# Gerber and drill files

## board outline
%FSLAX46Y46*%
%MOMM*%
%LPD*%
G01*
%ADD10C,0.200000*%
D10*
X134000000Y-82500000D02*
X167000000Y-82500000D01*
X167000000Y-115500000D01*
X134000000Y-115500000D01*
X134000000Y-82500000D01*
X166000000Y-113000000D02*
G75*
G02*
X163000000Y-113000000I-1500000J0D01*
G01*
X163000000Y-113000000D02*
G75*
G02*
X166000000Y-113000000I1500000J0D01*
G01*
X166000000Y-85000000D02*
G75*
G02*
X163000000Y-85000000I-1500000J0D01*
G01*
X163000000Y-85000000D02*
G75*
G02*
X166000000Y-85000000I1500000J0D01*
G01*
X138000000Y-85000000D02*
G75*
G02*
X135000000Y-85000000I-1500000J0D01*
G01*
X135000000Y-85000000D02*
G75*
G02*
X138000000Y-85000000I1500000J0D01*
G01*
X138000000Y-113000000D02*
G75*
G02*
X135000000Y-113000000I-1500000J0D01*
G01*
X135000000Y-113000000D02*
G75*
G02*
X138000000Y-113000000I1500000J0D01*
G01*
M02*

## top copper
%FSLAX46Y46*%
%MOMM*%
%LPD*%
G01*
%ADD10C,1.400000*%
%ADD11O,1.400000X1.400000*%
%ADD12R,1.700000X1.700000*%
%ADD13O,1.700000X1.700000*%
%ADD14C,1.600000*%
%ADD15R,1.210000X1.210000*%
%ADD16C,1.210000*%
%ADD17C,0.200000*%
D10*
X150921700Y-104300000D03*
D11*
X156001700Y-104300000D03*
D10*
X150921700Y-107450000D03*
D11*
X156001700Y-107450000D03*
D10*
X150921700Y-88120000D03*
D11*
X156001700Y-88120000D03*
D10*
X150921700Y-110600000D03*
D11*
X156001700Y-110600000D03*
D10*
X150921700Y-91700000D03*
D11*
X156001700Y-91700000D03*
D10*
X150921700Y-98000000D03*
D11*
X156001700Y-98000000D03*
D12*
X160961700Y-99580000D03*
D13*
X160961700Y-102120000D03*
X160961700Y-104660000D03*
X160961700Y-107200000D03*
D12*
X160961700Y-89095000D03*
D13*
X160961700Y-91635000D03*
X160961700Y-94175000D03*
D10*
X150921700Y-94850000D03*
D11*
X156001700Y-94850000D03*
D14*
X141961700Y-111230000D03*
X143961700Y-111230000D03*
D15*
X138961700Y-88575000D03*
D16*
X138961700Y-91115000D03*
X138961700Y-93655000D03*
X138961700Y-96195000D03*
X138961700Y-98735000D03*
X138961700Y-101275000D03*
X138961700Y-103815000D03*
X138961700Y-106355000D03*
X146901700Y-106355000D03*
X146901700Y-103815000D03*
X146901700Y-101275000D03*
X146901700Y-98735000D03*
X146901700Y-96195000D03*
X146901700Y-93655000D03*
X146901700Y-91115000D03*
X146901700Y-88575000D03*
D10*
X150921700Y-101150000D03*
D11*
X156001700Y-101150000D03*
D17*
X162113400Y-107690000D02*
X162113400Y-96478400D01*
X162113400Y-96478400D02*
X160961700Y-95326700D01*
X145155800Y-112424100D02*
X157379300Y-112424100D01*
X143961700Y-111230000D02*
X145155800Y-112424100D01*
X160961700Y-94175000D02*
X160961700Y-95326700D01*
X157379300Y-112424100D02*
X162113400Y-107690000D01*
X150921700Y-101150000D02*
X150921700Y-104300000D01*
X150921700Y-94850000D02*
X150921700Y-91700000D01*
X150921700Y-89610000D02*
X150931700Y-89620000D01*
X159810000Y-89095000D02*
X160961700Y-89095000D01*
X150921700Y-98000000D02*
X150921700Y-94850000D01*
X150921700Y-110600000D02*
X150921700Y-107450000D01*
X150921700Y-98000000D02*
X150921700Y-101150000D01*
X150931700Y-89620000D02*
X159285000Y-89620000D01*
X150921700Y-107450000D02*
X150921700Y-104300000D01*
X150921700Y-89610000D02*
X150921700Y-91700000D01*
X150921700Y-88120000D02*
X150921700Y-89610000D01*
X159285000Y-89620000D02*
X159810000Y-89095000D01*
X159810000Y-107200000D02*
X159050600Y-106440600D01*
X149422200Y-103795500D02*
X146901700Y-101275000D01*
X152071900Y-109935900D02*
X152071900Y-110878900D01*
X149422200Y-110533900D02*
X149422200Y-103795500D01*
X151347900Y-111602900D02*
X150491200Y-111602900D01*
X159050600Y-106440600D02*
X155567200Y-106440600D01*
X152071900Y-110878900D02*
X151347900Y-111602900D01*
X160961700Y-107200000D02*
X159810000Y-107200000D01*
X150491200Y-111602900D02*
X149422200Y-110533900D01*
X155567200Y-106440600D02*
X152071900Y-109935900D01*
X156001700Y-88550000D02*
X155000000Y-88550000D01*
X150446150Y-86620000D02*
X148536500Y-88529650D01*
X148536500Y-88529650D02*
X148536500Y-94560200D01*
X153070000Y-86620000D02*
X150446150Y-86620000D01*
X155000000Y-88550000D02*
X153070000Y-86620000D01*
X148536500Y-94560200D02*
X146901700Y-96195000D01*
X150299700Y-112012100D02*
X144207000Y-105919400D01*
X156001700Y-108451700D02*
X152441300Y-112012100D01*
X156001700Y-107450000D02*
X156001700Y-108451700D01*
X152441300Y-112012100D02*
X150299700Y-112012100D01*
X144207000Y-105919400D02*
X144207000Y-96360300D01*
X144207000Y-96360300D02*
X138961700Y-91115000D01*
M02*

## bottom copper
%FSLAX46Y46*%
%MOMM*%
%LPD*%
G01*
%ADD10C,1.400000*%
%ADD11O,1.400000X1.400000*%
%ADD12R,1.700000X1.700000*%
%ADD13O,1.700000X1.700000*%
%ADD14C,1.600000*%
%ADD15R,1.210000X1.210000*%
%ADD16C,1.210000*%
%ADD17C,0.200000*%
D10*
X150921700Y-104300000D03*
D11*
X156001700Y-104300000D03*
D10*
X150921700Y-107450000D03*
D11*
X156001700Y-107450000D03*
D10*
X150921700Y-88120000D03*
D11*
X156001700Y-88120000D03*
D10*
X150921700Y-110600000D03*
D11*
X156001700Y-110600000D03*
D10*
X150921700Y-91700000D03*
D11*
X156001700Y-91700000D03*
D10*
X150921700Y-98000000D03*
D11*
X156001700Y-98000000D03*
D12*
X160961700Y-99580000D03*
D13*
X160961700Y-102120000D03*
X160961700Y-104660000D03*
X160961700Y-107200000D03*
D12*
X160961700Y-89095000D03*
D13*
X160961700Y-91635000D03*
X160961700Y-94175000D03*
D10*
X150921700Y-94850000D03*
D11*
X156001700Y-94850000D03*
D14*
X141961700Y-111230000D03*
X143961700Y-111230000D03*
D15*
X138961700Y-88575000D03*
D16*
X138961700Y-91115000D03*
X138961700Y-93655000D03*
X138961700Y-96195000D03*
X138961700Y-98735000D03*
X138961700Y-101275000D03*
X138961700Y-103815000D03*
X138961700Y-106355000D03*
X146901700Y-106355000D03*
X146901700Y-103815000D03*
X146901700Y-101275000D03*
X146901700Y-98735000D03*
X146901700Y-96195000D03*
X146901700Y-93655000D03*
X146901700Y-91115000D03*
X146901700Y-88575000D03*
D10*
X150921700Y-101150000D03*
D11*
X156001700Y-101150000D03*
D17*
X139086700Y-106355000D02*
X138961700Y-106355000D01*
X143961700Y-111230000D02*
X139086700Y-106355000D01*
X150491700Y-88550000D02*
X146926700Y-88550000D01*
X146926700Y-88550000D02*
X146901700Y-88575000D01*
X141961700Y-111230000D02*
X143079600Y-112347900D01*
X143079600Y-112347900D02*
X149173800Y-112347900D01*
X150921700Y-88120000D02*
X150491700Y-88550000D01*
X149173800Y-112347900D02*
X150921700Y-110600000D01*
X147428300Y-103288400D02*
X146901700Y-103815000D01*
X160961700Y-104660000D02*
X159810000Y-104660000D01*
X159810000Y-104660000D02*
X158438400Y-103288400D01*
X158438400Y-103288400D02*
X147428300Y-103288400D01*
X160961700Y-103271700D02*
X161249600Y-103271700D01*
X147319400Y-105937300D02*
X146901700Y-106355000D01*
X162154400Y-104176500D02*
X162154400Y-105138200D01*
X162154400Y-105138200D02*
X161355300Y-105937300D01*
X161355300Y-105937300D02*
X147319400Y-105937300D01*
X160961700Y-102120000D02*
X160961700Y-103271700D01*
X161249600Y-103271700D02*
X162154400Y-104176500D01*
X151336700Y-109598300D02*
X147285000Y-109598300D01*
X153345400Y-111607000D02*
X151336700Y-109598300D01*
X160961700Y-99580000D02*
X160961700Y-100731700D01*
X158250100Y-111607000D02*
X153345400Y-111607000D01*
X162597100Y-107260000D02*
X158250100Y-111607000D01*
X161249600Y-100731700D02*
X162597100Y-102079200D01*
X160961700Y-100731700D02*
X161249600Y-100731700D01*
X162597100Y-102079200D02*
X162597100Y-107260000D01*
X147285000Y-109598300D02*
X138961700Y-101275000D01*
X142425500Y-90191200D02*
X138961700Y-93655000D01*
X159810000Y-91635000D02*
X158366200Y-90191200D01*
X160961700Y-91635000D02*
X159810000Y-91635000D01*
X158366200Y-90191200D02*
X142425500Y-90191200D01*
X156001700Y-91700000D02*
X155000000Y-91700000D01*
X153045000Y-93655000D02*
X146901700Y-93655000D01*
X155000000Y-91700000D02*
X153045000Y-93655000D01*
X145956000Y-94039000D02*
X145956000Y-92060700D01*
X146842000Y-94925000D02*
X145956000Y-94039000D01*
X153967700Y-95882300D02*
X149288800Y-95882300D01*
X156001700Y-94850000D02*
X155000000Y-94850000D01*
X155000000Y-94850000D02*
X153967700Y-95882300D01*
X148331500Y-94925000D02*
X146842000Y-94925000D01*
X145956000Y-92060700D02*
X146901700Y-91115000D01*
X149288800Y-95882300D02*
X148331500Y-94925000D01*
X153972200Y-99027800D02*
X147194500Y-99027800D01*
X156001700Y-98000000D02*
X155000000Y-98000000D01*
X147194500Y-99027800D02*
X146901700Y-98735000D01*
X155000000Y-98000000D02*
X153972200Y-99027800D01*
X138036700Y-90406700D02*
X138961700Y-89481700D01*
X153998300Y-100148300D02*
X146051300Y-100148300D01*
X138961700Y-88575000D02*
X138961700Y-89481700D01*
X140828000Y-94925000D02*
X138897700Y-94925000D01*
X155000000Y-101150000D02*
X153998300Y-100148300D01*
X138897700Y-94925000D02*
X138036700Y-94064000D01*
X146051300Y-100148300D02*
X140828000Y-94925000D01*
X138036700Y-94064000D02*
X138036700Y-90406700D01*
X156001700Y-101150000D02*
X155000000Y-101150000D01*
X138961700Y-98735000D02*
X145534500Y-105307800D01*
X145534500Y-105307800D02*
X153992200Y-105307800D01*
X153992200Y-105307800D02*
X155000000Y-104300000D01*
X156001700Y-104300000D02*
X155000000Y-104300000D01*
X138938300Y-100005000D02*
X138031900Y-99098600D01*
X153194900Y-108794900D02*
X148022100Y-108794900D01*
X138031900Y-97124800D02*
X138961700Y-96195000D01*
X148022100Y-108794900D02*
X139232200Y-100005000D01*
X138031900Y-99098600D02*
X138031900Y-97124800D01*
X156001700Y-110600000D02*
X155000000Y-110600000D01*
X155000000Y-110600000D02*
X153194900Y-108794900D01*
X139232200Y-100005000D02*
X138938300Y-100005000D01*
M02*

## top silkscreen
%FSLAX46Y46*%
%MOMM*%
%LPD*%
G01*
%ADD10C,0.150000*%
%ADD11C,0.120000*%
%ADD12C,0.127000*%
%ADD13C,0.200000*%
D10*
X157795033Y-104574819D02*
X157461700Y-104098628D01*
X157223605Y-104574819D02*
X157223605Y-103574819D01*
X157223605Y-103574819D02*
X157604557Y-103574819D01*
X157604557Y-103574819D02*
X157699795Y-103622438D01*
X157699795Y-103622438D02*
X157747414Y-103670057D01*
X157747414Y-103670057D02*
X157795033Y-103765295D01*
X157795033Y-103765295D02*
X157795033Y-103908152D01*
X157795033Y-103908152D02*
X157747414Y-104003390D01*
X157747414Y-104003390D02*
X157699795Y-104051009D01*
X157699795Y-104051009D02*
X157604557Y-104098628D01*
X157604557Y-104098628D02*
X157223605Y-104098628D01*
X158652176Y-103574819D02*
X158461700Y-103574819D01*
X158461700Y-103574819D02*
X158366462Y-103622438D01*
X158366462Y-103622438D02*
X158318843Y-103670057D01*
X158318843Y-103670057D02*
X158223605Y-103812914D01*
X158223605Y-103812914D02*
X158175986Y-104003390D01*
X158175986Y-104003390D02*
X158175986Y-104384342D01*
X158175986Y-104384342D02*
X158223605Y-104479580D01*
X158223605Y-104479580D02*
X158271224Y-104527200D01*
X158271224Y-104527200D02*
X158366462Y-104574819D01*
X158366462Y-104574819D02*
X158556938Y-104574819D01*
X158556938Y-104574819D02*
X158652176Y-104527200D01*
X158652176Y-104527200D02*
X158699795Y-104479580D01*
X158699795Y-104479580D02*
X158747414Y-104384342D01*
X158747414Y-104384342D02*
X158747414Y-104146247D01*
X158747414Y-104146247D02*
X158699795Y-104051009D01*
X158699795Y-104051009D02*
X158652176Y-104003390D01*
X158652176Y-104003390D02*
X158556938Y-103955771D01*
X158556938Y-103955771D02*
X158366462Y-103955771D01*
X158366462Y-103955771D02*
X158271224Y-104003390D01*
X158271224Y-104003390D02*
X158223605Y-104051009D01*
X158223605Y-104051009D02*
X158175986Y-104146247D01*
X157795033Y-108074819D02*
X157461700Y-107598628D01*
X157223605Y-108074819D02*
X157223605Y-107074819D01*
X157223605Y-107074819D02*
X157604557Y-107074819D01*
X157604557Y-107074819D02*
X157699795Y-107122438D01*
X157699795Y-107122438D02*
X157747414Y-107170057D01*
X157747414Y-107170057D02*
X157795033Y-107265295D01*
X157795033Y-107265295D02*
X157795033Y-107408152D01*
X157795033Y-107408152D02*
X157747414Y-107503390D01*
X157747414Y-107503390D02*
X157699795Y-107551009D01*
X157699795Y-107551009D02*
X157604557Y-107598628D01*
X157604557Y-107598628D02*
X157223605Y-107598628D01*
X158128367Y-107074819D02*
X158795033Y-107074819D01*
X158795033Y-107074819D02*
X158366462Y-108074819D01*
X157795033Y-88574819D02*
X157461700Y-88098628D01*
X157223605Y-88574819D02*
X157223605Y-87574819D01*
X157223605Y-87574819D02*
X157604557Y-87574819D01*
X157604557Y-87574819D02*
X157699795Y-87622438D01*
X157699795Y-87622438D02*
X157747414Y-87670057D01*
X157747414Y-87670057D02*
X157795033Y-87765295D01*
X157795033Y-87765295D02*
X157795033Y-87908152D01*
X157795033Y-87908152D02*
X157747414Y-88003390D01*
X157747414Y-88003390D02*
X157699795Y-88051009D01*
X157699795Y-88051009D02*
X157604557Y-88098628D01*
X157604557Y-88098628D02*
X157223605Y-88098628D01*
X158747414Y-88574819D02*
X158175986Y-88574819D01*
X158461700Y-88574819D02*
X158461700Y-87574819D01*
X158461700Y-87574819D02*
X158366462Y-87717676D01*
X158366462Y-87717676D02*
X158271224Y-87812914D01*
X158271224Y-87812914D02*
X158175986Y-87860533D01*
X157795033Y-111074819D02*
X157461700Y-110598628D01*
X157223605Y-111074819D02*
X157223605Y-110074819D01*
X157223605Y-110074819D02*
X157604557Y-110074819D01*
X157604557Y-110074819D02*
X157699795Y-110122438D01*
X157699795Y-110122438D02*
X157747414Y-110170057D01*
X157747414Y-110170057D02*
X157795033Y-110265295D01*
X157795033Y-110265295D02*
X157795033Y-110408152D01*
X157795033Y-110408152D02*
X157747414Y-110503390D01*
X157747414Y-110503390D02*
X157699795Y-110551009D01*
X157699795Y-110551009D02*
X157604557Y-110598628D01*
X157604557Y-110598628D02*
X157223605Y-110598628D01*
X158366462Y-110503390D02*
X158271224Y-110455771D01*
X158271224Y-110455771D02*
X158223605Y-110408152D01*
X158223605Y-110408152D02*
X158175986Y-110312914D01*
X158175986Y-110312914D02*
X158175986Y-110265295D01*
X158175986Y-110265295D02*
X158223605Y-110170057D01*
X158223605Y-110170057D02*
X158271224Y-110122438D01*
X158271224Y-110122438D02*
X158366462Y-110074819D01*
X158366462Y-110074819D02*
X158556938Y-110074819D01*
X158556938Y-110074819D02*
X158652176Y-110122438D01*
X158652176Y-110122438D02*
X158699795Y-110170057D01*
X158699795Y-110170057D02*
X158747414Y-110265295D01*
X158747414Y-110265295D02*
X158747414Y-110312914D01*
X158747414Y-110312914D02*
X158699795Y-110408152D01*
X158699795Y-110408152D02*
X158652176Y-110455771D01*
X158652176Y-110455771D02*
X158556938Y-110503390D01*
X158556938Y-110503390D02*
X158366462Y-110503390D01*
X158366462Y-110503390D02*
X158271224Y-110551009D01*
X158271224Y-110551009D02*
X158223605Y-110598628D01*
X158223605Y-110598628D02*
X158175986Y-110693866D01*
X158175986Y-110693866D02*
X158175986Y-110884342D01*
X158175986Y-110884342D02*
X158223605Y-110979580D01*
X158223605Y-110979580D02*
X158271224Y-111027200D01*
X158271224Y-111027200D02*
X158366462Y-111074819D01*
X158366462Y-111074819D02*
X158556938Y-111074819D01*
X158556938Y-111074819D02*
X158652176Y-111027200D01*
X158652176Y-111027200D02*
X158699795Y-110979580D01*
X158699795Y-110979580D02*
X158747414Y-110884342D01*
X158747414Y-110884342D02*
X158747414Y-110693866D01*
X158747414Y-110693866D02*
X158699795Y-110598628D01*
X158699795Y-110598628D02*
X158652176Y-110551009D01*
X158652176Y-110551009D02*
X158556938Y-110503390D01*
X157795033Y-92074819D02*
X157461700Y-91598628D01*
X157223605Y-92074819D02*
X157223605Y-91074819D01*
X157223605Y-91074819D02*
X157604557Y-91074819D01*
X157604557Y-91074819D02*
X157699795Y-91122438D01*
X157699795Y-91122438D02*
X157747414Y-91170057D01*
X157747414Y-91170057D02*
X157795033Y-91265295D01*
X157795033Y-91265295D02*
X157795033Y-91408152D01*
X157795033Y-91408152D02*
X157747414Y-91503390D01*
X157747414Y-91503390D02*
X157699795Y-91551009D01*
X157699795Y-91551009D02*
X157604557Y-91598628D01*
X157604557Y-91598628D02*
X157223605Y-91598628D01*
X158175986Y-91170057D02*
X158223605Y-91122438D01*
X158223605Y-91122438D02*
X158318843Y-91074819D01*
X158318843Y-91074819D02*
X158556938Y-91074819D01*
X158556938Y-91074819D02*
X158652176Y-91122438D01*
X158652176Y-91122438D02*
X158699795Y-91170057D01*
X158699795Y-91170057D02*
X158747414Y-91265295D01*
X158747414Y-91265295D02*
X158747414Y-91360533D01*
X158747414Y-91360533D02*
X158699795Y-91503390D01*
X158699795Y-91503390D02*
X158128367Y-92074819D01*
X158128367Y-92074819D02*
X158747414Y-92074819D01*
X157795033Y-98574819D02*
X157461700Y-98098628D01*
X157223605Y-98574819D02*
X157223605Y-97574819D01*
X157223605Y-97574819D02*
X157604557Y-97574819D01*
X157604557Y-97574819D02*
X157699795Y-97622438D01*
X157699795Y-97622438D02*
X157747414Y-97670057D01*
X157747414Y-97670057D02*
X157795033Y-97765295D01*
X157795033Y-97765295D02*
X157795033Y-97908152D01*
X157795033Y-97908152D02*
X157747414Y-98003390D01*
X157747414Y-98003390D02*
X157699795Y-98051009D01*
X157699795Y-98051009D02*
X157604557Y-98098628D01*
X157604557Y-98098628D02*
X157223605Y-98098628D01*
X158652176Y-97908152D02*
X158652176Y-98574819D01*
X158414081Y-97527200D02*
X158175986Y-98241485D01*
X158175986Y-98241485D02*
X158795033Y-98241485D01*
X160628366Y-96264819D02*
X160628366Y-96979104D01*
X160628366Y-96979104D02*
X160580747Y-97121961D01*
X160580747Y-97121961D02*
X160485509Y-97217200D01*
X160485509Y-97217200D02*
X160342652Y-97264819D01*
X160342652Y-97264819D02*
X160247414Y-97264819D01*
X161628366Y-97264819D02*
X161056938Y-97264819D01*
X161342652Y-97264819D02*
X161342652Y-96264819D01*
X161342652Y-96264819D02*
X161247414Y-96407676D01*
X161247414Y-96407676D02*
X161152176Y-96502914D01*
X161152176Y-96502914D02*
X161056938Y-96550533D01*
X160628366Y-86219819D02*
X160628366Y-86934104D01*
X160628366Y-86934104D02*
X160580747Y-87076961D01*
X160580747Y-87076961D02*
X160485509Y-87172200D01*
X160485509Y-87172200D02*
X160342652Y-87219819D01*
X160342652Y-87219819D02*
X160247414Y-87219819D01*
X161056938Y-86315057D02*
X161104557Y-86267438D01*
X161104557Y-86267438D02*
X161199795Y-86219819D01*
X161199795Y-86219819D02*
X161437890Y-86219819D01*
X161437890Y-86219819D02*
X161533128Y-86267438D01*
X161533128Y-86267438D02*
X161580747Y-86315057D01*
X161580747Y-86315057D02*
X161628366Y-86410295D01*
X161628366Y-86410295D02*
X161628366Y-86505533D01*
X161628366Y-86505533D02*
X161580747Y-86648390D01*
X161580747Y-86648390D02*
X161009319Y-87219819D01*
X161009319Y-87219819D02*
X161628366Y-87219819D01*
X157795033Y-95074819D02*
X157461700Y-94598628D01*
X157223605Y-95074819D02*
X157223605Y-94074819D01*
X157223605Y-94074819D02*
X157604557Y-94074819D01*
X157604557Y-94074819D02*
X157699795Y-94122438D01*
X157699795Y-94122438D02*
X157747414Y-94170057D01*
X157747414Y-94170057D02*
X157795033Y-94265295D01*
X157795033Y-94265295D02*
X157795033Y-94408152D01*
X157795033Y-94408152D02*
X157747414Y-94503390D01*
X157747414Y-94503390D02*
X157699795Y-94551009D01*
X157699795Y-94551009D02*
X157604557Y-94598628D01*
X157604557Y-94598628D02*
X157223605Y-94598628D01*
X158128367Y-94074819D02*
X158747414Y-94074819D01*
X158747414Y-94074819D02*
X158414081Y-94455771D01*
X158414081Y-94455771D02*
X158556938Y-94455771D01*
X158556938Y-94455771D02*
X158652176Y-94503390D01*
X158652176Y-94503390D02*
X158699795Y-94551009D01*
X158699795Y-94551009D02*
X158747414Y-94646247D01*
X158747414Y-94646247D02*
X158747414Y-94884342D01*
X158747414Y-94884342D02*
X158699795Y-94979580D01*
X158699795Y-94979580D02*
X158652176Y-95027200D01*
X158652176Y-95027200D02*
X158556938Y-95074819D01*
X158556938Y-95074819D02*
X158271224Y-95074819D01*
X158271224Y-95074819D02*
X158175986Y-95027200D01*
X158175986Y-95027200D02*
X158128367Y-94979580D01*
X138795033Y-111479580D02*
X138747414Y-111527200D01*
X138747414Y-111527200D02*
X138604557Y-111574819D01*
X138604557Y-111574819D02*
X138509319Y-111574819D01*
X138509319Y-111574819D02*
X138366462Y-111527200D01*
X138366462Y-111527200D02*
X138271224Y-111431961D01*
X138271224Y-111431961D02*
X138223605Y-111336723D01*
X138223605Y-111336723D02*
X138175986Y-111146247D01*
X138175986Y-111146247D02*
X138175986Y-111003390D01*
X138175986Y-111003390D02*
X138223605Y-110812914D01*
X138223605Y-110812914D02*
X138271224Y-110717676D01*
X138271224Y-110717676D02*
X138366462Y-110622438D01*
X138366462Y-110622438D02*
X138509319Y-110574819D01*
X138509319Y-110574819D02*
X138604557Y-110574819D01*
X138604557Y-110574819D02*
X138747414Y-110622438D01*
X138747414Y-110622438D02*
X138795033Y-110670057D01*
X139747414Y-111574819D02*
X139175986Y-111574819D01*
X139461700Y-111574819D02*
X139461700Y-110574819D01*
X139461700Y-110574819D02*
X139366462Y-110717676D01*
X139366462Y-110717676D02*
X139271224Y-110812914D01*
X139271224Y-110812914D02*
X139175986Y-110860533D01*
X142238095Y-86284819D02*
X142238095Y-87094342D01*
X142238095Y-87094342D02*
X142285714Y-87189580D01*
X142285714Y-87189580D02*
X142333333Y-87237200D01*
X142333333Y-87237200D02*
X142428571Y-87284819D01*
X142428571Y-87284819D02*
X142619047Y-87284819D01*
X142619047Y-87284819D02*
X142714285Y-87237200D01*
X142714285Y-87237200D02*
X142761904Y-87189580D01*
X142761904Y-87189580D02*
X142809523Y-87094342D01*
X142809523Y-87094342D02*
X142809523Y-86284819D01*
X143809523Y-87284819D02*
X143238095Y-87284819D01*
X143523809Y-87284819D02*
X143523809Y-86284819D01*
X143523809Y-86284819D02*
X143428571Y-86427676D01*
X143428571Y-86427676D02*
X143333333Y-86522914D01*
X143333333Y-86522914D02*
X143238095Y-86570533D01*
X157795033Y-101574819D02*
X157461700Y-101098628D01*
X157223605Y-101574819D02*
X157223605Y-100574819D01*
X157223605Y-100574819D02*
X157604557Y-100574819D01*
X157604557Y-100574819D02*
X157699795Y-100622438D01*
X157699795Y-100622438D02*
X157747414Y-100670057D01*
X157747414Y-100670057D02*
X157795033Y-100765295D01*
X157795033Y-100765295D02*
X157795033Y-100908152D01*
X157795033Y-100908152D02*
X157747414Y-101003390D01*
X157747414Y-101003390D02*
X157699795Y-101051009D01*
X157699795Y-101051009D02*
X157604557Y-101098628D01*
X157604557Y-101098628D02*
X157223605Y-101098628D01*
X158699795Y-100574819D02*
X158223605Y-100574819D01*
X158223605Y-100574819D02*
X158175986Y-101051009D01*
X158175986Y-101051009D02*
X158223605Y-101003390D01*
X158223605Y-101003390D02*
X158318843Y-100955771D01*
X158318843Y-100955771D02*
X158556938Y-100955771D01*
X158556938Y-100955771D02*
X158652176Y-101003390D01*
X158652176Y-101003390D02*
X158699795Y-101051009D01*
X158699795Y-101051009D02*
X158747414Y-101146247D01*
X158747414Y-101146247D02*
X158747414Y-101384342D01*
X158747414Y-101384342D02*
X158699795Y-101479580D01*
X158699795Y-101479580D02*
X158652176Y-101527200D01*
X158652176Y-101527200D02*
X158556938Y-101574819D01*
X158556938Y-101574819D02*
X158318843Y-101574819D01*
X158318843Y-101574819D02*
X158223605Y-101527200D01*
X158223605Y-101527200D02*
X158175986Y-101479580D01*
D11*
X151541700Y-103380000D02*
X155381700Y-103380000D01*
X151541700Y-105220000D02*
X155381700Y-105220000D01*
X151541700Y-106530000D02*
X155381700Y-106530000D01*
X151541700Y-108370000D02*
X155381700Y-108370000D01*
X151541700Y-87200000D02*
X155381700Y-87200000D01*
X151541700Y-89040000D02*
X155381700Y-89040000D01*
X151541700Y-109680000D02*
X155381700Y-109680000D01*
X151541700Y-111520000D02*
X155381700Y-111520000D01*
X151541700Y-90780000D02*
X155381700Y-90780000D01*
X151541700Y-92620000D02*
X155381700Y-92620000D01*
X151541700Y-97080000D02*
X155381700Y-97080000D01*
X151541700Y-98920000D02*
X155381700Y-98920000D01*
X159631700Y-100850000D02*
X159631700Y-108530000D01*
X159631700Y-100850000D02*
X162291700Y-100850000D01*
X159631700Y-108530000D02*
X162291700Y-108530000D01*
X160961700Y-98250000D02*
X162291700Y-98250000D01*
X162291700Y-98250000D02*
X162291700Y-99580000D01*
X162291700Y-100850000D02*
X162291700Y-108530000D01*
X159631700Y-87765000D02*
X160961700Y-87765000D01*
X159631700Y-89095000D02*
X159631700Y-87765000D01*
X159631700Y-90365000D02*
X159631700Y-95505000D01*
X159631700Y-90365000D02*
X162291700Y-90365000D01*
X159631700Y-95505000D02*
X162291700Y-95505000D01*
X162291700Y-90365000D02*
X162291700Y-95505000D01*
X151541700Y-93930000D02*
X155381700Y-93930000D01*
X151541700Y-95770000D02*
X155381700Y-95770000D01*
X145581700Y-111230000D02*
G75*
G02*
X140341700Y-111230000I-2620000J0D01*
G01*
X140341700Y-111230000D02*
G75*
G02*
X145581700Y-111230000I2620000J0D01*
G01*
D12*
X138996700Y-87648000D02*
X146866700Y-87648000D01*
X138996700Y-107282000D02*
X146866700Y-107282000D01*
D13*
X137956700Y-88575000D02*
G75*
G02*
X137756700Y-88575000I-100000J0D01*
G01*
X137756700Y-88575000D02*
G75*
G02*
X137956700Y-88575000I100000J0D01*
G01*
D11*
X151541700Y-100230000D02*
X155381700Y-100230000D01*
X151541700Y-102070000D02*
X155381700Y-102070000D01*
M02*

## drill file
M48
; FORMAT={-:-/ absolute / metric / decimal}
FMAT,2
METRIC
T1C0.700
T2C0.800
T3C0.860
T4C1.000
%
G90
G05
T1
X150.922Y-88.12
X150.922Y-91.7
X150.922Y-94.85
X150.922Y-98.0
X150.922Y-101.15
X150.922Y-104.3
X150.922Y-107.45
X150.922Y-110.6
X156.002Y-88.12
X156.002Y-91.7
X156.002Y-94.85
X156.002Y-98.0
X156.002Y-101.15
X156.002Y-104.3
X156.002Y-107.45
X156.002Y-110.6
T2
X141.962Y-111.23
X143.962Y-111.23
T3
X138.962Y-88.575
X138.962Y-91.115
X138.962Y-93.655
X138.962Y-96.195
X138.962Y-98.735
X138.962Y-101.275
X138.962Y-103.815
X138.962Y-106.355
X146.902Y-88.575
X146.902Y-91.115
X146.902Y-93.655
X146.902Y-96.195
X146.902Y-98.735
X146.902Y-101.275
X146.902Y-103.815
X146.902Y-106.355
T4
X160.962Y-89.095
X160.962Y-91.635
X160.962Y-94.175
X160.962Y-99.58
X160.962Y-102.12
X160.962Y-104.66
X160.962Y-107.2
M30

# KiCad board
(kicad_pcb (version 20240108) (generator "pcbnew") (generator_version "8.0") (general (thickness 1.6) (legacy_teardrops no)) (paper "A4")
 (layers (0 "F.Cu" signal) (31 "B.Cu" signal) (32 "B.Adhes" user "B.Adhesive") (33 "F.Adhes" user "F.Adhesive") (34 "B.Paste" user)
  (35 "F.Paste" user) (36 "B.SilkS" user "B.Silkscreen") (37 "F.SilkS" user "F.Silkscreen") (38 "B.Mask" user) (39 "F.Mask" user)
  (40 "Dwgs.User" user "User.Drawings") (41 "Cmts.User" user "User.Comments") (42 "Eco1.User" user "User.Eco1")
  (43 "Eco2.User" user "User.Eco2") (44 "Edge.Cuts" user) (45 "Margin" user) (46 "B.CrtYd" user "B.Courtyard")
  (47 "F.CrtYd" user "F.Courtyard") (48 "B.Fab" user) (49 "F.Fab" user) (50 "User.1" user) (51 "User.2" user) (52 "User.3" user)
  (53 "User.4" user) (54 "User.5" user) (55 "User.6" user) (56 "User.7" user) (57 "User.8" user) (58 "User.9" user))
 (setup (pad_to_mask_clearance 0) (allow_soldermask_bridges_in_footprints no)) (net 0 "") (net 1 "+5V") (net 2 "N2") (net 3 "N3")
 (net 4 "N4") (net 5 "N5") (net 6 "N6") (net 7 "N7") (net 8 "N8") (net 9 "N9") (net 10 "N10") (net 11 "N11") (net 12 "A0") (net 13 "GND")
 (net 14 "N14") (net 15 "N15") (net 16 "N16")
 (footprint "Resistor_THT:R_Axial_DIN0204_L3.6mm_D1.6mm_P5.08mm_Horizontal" (layer "F.Cu") (at 150.9217 104.3)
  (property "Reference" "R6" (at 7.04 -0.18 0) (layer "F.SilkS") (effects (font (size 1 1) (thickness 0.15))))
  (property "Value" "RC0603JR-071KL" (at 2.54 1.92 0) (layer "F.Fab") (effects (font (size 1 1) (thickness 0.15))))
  (fp_line (start 0.62 -0.92) (end 4.46 -0.92) (stroke (width 0.12) (type solid)) (layer "F.SilkS"))
  (fp_line (start 0.62 0.92) (end 4.46 0.92) (stroke (width 0.12) (type solid)) (layer "F.SilkS"))
  (pad "1" thru_hole circle (at 0 0) (size 1.4 1.4) (drill 0.7) (layers "*.Cu" "*.Mask") (remove_unused_layers no) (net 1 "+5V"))
  (pad "2" thru_hole oval (at 5.08 0) (size 1.4 1.4) (drill 0.7) (layers "*.Cu" "*.Mask") (remove_unused_layers no) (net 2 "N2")))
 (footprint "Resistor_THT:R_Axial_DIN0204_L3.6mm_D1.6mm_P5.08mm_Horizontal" (layer "F.Cu") (at 150.9217 107.45)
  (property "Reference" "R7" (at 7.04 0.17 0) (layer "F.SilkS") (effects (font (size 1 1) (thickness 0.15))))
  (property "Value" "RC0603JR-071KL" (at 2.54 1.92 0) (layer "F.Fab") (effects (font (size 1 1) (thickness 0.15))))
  (fp_line (start 0.62 -0.92) (end 4.46 -0.92) (stroke (width 0.12) (type solid)) (layer "F.SilkS"))
  (fp_line (start 0.62 0.92) (end 4.46 0.92) (stroke (width 0.12) (type solid)) (layer "F.SilkS"))
  (pad "1" thru_hole circle (at 0 0) (size 1.4 1.4) (drill 0.7) (layers "*.Cu" "*.Mask") (remove_unused_layers no) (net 1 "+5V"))
  (pad "2" thru_hole oval (at 5.08 0) (size 1.4 1.4) (drill 0.7) (layers "*.Cu" "*.Mask") (remove_unused_layers no) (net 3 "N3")))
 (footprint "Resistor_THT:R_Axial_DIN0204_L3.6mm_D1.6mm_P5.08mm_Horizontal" (layer "F.Cu") (at 150.9217 88.12)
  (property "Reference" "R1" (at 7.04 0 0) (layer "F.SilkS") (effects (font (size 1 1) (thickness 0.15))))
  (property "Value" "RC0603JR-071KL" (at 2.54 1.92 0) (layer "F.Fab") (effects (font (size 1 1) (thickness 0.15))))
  (fp_line (start 0.62 -0.92) (end 4.46 -0.92) (stroke (width 0.12) (type solid)) (layer "F.SilkS"))
  (fp_line (start 0.62 0.92) (end 4.46 0.92) (stroke (width 0.12) (type solid)) (layer "F.SilkS"))
  (pad "1" thru_hole circle (at 0 0) (size 1.4 1.4) (drill 0.7) (layers "*.Cu" "*.Mask") (remove_unused_layers no) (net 1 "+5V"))
  (pad "2" thru_hole oval (at 5.08 0) (size 1.4 1.4) (drill 0.7) (layers "*.Cu" "*.Mask") (remove_unused_layers no) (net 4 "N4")))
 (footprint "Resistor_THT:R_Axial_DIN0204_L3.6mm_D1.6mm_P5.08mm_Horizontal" (layer "F.Cu") (at 150.9217 110.6)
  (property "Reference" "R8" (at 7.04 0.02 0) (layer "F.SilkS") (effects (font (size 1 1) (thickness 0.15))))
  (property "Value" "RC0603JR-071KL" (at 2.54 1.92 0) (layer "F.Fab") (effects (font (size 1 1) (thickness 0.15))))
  (fp_line (start 0.62 -0.92) (end 4.46 -0.92) (stroke (width 0.12) (type solid)) (layer "F.SilkS"))
  (fp_line (start 0.62 0.92) (end 4.46 0.92) (stroke (width 0.12) (type solid)) (layer "F.SilkS"))
  (pad "1" thru_hole circle (at 0 0) (size 1.4 1.4) (drill 0.7) (layers "*.Cu" "*.Mask") (remove_unused_layers no) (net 1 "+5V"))
  (pad "2" thru_hole oval (at 5.08 0) (size 1.4 1.4) (drill 0.7) (layers "*.Cu" "*.Mask") (remove_unused_layers no) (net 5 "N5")))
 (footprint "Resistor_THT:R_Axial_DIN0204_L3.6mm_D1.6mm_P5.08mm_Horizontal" (layer "F.Cu") (at 150.9217 91.7)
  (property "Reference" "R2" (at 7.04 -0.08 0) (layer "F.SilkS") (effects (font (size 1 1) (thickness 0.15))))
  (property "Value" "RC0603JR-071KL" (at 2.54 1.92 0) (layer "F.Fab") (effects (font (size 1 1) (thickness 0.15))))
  (fp_line (start 0.62 -0.92) (end 4.46 -0.92) (stroke (width 0.12) (type solid)) (layer "F.SilkS"))
  (fp_line (start 0.62 0.92) (end 4.46 0.92) (stroke (width 0.12) (type solid)) (layer "F.SilkS"))
  (pad "1" thru_hole circle (at 0 0) (size 1.4 1.4) (drill 0.7) (layers "*.Cu" "*.Mask") (remove_unused_layers no) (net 1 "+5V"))
  (pad "2" thru_hole oval (at 5.08 0) (size 1.4 1.4) (drill 0.7) (layers "*.Cu" "*.Mask") (remove_unused_layers no) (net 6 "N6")))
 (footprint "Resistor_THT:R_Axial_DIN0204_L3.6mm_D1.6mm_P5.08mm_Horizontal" (layer "F.Cu") (at 150.9217 98)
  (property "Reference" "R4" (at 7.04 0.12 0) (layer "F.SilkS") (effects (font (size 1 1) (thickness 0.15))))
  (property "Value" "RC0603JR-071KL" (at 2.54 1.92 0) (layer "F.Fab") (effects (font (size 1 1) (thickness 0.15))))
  (fp_line (start 0.62 -0.92) (end 4.46 -0.92) (stroke (width 0.12) (type solid)) (layer "F.SilkS"))
  (fp_line (start 0.62 0.92) (end 4.46 0.92) (stroke (width 0.12) (type solid)) (layer "F.SilkS"))
  (pad "1" thru_hole circle (at 0 0) (size 1.4 1.4) (drill 0.7) (layers "*.Cu" "*.Mask") (remove_unused_layers no) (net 1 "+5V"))
  (pad "2" thru_hole oval (at 5.08 0) (size 1.4 1.4) (drill 0.7) (layers "*.Cu" "*.Mask") (remove_unused_layers no) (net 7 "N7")))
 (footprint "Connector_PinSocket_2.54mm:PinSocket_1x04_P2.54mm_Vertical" (layer "F.Cu") (at 160.9617 99.58)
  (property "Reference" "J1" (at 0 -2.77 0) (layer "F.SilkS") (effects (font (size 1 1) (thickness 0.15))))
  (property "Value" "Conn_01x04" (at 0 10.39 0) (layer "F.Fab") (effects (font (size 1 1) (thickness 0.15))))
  (fp_line (start -1.33 1.27) (end -1.33 8.95) (stroke (width 0.12) (type solid)) (layer "F.SilkS"))
  (fp_line (start -1.33 1.27) (end 1.33 1.27) (stroke (width 0.12) (type solid)) (layer "F.SilkS"))
  (fp_line (start -1.33 8.95) (end 1.33 8.95) (stroke (width 0.12) (type solid)) (layer "F.SilkS"))
  (fp_line (start 0 -1.33) (end 1.33 -1.33) (stroke (width 0.12) (type solid)) (layer "F.SilkS"))
  (fp_line (start 1.33 -1.33) (end 1.33 0) (stroke (width 0.12) (type solid)) (layer "F.SilkS"))
  (fp_line (start 1.33 1.27) (end 1.33 8.95) (stroke (width 0.12) (type solid)) (layer "F.SilkS"))
  (pad "1" thru_hole rect (at 0 0) (size 1.7 1.7) (drill 1) (layers "*.Cu" "*.Mask") (remove_unused_layers no) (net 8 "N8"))
  (pad "2" thru_hole oval (at 0 2.54) (size 1.7 1.7) (drill 1) (layers "*.Cu" "*.Mask") (remove_unused_layers no) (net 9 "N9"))
  (pad "3" thru_hole oval (at 0 5.08) (size 1.7 1.7) (drill 1) (layers "*.Cu" "*.Mask") (remove_unused_layers no) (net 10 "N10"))
  (pad "4" thru_hole oval (at 0 7.62) (size 1.7 1.7) (drill 1) (layers "*.Cu" "*.Mask") (remove_unused_layers no) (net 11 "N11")))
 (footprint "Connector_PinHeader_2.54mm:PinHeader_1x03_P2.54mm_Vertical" (layer "F.Cu") (at 160.9617 89.095)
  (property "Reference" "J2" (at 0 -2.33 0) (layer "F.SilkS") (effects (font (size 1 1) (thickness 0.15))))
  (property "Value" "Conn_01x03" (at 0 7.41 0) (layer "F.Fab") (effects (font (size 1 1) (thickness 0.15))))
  (fp_line (start -1.33 -1.33) (end 0 -1.33) (stroke (width 0.12) (type solid)) (layer "F.SilkS"))
  (fp_line (start -1.33 0) (end -1.33 -1.33) (stroke (width 0.12) (type solid)) (layer "F.SilkS"))
  (fp_line (start -1.33 1.27) (end -1.33 6.41) (stroke (width 0.12) (type solid)) (layer "F.SilkS"))
  (fp_line (start -1.33 1.27) (end 1.33 1.27) (stroke (width 0.12) (type solid)) (layer "F.SilkS"))
  (fp_line (start -1.33 6.41) (end 1.33 6.41) (stroke (width 0.12) (type solid)) (layer "F.SilkS"))
  (fp_line (start 1.33 1.27) (end 1.33 6.41) (stroke (width 0.12) (type solid)) (layer "F.SilkS"))
  (pad "1" thru_hole rect (at 0 0) (size 1.7 1.7) (drill 1) (layers "*.Cu" "*.Mask") (remove_unused_layers no) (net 1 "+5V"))
  (pad "2" thru_hole oval (at 0 2.54) (size 1.7 1.7) (drill 1) (layers "*.Cu" "*.Mask") (remove_unused_layers no) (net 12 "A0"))
  (pad "3" thru_hole oval (at 0 5.08) (size 1.7 1.7) (drill 1) (layers "*.Cu" "*.Mask") (remove_unused_layers no) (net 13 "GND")))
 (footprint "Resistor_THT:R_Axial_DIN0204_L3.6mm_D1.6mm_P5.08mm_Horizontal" (layer "F.Cu") (at 150.9217 94.85)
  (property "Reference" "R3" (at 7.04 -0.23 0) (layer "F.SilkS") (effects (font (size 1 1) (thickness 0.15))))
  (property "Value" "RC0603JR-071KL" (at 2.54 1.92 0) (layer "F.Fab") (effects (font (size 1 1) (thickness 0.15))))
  (fp_line (start 0.62 -0.92) (end 4.46 -0.92) (stroke (width 0.12) (type solid)) (layer "F.SilkS"))
  (fp_line (start 0.62 0.92) (end 4.46 0.92) (stroke (width 0.12) (type solid)) (layer "F.SilkS"))
  (pad "1" thru_hole circle (at 0 0) (size 1.4 1.4) (drill 0.7) (layers "*.Cu" "*.Mask") (remove_unused_layers no) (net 1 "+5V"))
  (pad "2" thru_hole oval (at 5.08 0) (size 1.4 1.4) (drill 0.7) (layers "*.Cu" "*.Mask") (remove_unused_layers no) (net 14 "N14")))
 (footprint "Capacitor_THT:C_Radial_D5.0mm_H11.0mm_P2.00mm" (layer "F.Cu") (at 141.9617 111.23)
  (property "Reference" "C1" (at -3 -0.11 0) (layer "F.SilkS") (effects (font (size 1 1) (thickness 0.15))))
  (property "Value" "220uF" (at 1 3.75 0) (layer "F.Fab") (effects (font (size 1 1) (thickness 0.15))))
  (fp_circle (center 1 0) (end 3.62 0) (stroke (width 0.12) (type solid)) (fill none) (layer "F.SilkS"))
  (pad "1" thru_hole circle (at 0 0) (size 1.6 1.6) (drill 0.8) (layers "*.Cu" "*.Mask") (remove_unused_layers no) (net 1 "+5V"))
  (pad "2" thru_hole circle (at 2 0) (size 1.6 1.6) (drill 0.8) (layers "*.Cu" "*.Mask") (remove_unused_layers no) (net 13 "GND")))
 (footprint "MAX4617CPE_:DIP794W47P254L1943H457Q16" (layer "F.Cu") (at 142.9317 97.465)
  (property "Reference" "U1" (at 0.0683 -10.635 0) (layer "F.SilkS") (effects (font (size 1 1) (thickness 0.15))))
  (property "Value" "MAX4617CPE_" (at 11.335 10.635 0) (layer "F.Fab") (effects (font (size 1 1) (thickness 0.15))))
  (fp_line (start -3.935 -9.817) (end 3.935 -9.817) (stroke (width 0.127) (type solid)) (layer "F.SilkS"))
  (fp_line (start -3.935 9.817) (end 3.935 9.817) (stroke (width 0.127) (type solid)) (layer "F.SilkS"))
  (fp_circle (center -5.075 -8.89) (end -4.975 -8.89) (stroke (width 0.2) (type solid)) (fill none) (layer "F.SilkS"))
  (pad "1" thru_hole rect (at -3.97 -8.89) (size 1.21 1.21) (drill 0.86) (layers "*.Cu" "*.Mask") (remove_unused_layers no) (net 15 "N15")
   (solder_mask_margin 0.102))
  (pad "2" thru_hole circle (at -3.97 -6.35) (size 1.21 1.21) (drill 0.86) (layers "*.Cu" "*.Mask") (remove_unused_layers no) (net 3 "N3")
   (solder_mask_margin 0.102))
  (pad "3" thru_hole circle (at -3.97 -3.81) (size 1.21 1.21) (drill 0.86) (layers "*.Cu" "*.Mask") (remove_unused_layers no) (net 12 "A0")
   (solder_mask_margin 0.102))
  (pad "4" thru_hole circle (at -3.97 -1.27) (size 1.21 1.21) (drill 0.86) (layers "*.Cu" "*.Mask") (remove_unused_layers no) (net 5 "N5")
   (solder_mask_margin 0.102))
  (pad "5" thru_hole circle (at -3.97 1.27) (size 1.21 1.21) (drill 0.86) (layers "*.Cu" "*.Mask") (remove_unused_layers no) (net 2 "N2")
   (solder_mask_margin 0.102))
  (pad "6" thru_hole circle (at -3.97 3.81) (size 1.21 1.21) (drill 0.86) (layers "*.Cu" "*.Mask") (remove_unused_layers no) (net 8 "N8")
   (solder_mask_margin 0.102))
  (pad "7" thru_hole circle (at -3.97 6.35) (size 1.21 1.21) (drill 0.86) (layers "*.Cu" "*.Mask") (remove_unused_layers no) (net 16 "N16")
   (solder_mask_margin 0.102))
  (pad "8" thru_hole circle (at -3.97 8.89) (size 1.21 1.21) (drill 0.86) (layers "*.Cu" "*.Mask") (remove_unused_layers no) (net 13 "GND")
   (solder_mask_margin 0.102))
  (pad "9" thru_hole circle (at 3.97 8.89) (size 1.21 1.21) (drill 0.86) (layers "*.Cu" "*.Mask") (remove_unused_layers no) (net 9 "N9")
   (solder_mask_margin 0.102))
  (pad "10" thru_hole circle (at 3.97 6.35) (size 1.21 1.21) (drill 0.86) (layers "*.Cu" "*.Mask") (remove_unused_layers no) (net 10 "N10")
   (solder_mask_margin 0.102))
  (pad "11" thru_hole circle (at 3.97 3.81) (size 1.21 1.21) (drill 0.86) (layers "*.Cu" "*.Mask") (remove_unused_layers no) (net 11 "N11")
   (solder_mask_margin 0.102))
  (pad "12" thru_hole circle (at 3.97 1.27) (size 1.21 1.21) (drill 0.86) (layers "*.Cu" "*.Mask") (remove_unused_layers no) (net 7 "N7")
   (solder_mask_margin 0.102))
  (pad "13" thru_hole circle (at 3.97 -1.27) (size 1.21 1.21) (drill 0.86) (layers "*.Cu" "*.Mask") (remove_unused_layers no) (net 4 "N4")
   (solder_mask_margin 0.102))
  (pad "14" thru_hole circle (at 3.97 -3.81) (size 1.21 1.21) (drill 0.86) (layers "*.Cu" "*.Mask") (remove_unused_layers no) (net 6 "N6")
   (solder_mask_margin 0.102))
  (pad "15" thru_hole circle (at 3.97 -6.35) (size 1.21 1.21) (drill 0.86) (layers "*.Cu" "*.Mask") (remove_unused_layers no) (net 14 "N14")
   (solder_mask_margin 0.102))
  (pad "16" thru_hole circle (at 3.97 -8.89) (size 1.21 1.21) (drill 0.86) (layers "*.Cu" "*.Mask") (remove_unused_layers no) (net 1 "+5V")
   (solder_mask_margin 0.102)))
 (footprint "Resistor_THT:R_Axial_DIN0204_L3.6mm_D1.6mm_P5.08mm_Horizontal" (layer "F.Cu") (at 150.9217 101.15)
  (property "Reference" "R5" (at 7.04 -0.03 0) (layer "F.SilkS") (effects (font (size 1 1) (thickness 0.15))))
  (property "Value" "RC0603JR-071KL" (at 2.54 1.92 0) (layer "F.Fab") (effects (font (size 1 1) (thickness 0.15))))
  (fp_line (start 0.62 -0.92) (end 4.46 -0.92) (stroke (width 0.12) (type solid)) (layer "F.SilkS"))
  (fp_line (start 0.62 0.92) (end 4.46 0.92) (stroke (width 0.12) (type solid)) (layer "F.SilkS"))
  (pad "1" thru_hole circle (at 0 0) (size 1.4 1.4) (drill 0.7) (layers "*.Cu" "*.Mask") (remove_unused_layers no) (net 1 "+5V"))
  (pad "2" thru_hole oval (at 5.08 0) (size 1.4 1.4) (drill 0.7) (layers "*.Cu" "*.Mask") (remove_unused_layers no) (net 15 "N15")))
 (gr_rect (start 134 82.5) (end 167 115.5) (stroke (width 0.2) (type default)) (fill none) (layer "Edge.Cuts"))
 (gr_circle (center 164.5 113) (end 166 113) (stroke (width 0.2) (type default)) (fill none) (layer "Edge.Cuts"))
 (gr_circle (center 164.5 85) (end 166 85) (stroke (width 0.2) (type default)) (fill none) (layer "Edge.Cuts"))
 (gr_circle (center 136.5 85) (end 138 85) (stroke (width 0.2) (type default)) (fill none) (layer "Edge.Cuts"))
 (gr_circle (center 136.5 113) (end 138 113) (stroke (width 0.2) (type default)) (fill none) (layer "Edge.Cuts"))
 (segment (start 162.1134 107.69) (end 162.1134 96.4784) (width 0.2) (layer "F.Cu") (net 13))
 (segment (start 162.1134 96.4784) (end 160.9617 95.3267) (width 0.2) (layer "F.Cu") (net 13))
 (segment (start 145.1558 112.4241) (end 157.3793 112.4241) (width 0.2) (layer "F.Cu") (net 13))
 (segment (start 143.9617 111.23) (end 145.1558 112.4241) (width 0.2) (layer "F.Cu") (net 13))
 (segment (start 160.9617 94.175) (end 160.9617 95.3267) (width 0.2) (layer "F.Cu") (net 13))
 (segment (start 157.3793 112.4241) (end 162.1134 107.69) (width 0.2) (layer "F.Cu") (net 13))
 (segment (start 139.0867 106.355) (end 138.9617 106.355) (width 0.2) (layer "B.Cu") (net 13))
 (segment (start 143.9617 111.23) (end 139.0867 106.355) (width 0.2) (layer "B.Cu") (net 13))
 (segment (start 150.9217 101.15) (end 150.9217 104.3) (width 0.2) (layer "F.Cu") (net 1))
 (segment (start 150.9217 94.85) (end 150.9217 91.7) (width 0.2) (layer "F.Cu") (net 1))
 (segment (start 150.9217 89.61) (end 150.9317 89.62) (width 0.2) (layer "F.Cu") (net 1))
 (segment (start 159.81 89.095) (end 160.9617 89.095) (width 0.2) (layer "F.Cu") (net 1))
 (segment (start 150.9217 98) (end 150.9217 94.85) (width 0.2) (layer "F.Cu") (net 1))
 (segment (start 150.9217 110.6) (end 150.9217 107.45) (width 0.2) (layer "F.Cu") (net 1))
 (segment (start 150.9217 98) (end 150.9217 101.15) (width 0.2) (layer "F.Cu") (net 1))
 (segment (start 150.9317 89.62) (end 159.285 89.62) (width 0.2) (layer "F.Cu") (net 1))
 (segment (start 150.9217 107.45) (end 150.9217 104.3) (width 0.2) (layer "F.Cu") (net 1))
 (segment (start 150.9217 89.61) (end 150.9217 91.7) (width 0.2) (layer "F.Cu") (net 1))
 (segment (start 150.9217 88.12) (end 150.9217 89.61) (width 0.2) (layer "F.Cu") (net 1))
 (segment (start 159.285 89.62) (end 159.81 89.095) (width 0.2) (layer "F.Cu") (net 1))
 (segment (start 150.4917 88.55) (end 146.9267 88.55) (width 0.2) (layer "B.Cu") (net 1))
 (segment (start 146.9267 88.55) (end 146.9017 88.575) (width 0.2) (layer "B.Cu") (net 1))
 (segment (start 141.9617 111.23) (end 143.0796 112.3479) (width 0.2) (layer "B.Cu") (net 1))
 (segment (start 143.0796 112.3479) (end 149.1738 112.3479) (width 0.2) (layer "B.Cu") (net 1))
 (segment (start 150.9217 88.12) (end 150.4917 88.55) (width 0.2) (layer "B.Cu") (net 1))
 (segment (start 149.1738 112.3479) (end 150.9217 110.6) (width 0.2) (layer "B.Cu") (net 1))
 (segment (start 159.81 107.2) (end 159.0506 106.4406) (width 0.2) (layer "F.Cu") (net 11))
 (segment (start 149.4222 103.7955) (end 146.9017 101.275) (width 0.2) (layer "F.Cu") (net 11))
 (segment (start 152.0719 109.9359) (end 152.0719 110.8789) (width 0.2) (layer "F.Cu") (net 11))
 (segment (start 149.4222 110.5339) (end 149.4222 103.7955) (width 0.2) (layer "F.Cu") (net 11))
 (segment (start 151.3479 111.6029) (end 150.4912 111.6029) (width 0.2) (layer "F.Cu") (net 11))
 (segment (start 159.0506 106.4406) (end 155.5672 106.4406) (width 0.2) (layer "F.Cu") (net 11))
 (segment (start 152.0719 110.8789) (end 151.3479 111.6029) (width 0.2) (layer "F.Cu") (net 11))
 (segment (start 160.9617 107.2) (end 159.81 107.2) (width 0.2) (layer "F.Cu") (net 11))
 (segment (start 150.4912 111.6029) (end 149.4222 110.5339) (width 0.2) (layer "F.Cu") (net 11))
 (segment (start 155.5672 106.4406) (end 152.0719 109.9359) (width 0.2) (layer "F.Cu") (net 11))
 (segment (start 147.4283 103.2884) (end 146.9017 103.815) (width 0.2) (layer "B.Cu") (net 10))
 (segment (start 160.9617 104.66) (end 159.81 104.66) (width 0.2) (layer "B.Cu") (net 10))
 (segment (start 159.81 104.66) (end 158.4384 103.2884) (width 0.2) (layer "B.Cu") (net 10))
 (segment (start 158.4384 103.2884) (end 147.4283 103.2884) (width 0.2) (layer "B.Cu") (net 10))
 (segment (start 160.9617 103.2717) (end 161.2496 103.2717) (width 0.2) (layer "B.Cu") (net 9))
 (segment (start 147.3194 105.9373) (end 146.9017 106.355) (width 0.2) (layer "B.Cu") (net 9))
 (segment (start 162.1544 104.1765) (end 162.1544 105.1382) (width 0.2) (layer "B.Cu") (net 9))
 (segment (start 162.1544 105.1382) (end 161.3553 105.9373) (width 0.2) (layer "B.Cu") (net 9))
 (segment (start 161.3553 105.9373) (end 147.3194 105.9373) (width 0.2) (layer "B.Cu") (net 9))
 (segment (start 160.9617 102.12) (end 160.9617 103.2717) (width 0.2) (layer "B.Cu") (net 9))
 (segment (start 161.2496 103.2717) (end 162.1544 104.1765) (width 0.2) (layer "B.Cu") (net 9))
 (segment (start 151.3367 109.5983) (end 147.285 109.5983) (width 0.2) (layer "B.Cu") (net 8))
 (segment (start 153.3454 111.607) (end 151.3367 109.5983) (width 0.2) (layer "B.Cu") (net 8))
 (segment (start 160.9617 99.58) (end 160.9617 100.7317) (width 0.2) (layer "B.Cu") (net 8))
 (segment (start 158.2501 111.607) (end 153.3454 111.607) (width 0.2) (layer "B.Cu") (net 8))
 (segment (start 162.5971 107.26) (end 158.2501 111.607) (width 0.2) (layer "B.Cu") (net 8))
 (segment (start 161.2496 100.7317) (end 162.5971 102.0792) (width 0.2) (layer "B.Cu") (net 8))
 (segment (start 160.9617 100.7317) (end 161.2496 100.7317) (width 0.2) (layer "B.Cu") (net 8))
 (segment (start 162.5971 102.0792) (end 162.5971 107.26) (width 0.2) (layer "B.Cu") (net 8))
 (segment (start 147.285 109.5983) (end 138.9617 101.275) (width 0.2) (layer "B.Cu") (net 8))
 (segment (start 142.4255 90.1912) (end 138.9617 93.655) (width 0.2) (layer "B.Cu") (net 12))
 (segment (start 159.81 91.635) (end 158.3662 90.1912) (width 0.2) (layer "B.Cu") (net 12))
 (segment (start 160.9617 91.635) (end 159.81 91.635) (width 0.2) (layer "B.Cu") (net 12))
 (segment (start 158.3662 90.1912) (end 142.4255 90.1912) (width 0.2) (layer "B.Cu") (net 12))
 (segment (start 156.0017 88.55) (end 155 88.55) (width 0.2) (layer "F.Cu") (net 4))
 (segment (start 150.44615 86.62) (end 148.5365 88.52965) (width 0.2) (layer "F.Cu") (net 4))
 (segment (start 148.5365 88.52965) (end 148.5365 94.5602) (width 0.2) (layer "F.Cu") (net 4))
 (segment (start 153.07 86.62) (end 150.44615 86.62) (width 0.2) (layer "F.Cu") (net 4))
 (segment (start 155 88.55) (end 153.07 86.62) (width 0.2) (layer "F.Cu") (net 4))
 (segment (start 148.5365 94.5602) (end 146.9017 96.195) (width 0.2) (layer "F.Cu") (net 4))
 (segment (start 156.0017 91.7) (end 155 91.7) (width 0.2) (layer "B.Cu") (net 6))
 (segment (start 153.045 93.655) (end 146.9017 93.655) (width 0.2) (layer "B.Cu") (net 6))
 (segment (start 155 91.7) (end 153.045 93.655) (width 0.2) (layer "B.Cu") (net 6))
 (segment (start 145.956 94.039) (end 145.956 92.0607) (width 0.2) (layer "B.Cu") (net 14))
 (segment (start 146.842 94.925) (end 145.956 94.039) (width 0.2) (layer "B.Cu") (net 14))
 (segment (start 153.9677 95.8823) (end 149.2888 95.8823) (width 0.2) (layer "B.Cu") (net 14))
 (segment (start 156.0017 94.85) (end 155 94.85) (width 0.2) (layer "B.Cu") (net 14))
 (segment (start 155 94.85) (end 153.9677 95.8823) (width 0.2) (layer "B.Cu") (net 14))
 (segment (start 148.3315 94.925) (end 146.842 94.925) (width 0.2) (layer "B.Cu") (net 14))
 (segment (start 145.956 92.0607) (end 146.9017 91.115) (width 0.2) (layer "B.Cu") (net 14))
 (segment (start 149.2888 95.8823) (end 148.3315 94.925) (width 0.2) (layer "B.Cu") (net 14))
 (segment (start 153.9722 99.0278) (end 147.1945 99.0278) (width 0.2) (layer "B.Cu") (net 7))
 (segment (start 156.0017 98) (end 155 98) (width 0.2) (layer "B.Cu") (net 7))
 (segment (start 147.1945 99.0278) (end 146.9017 98.735) (width 0.2) (layer "B.Cu") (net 7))
 (segment (start 155 98) (end 153.9722 99.0278) (width 0.2) (layer "B.Cu") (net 7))
 (segment (start 138.0367 90.4067) (end 138.9617 89.4817) (width 0.2) (layer "B.Cu") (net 15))
 (segment (start 153.9983 100.1483) (end 146.0513 100.1483) (width 0.2) (layer "B.Cu") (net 15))
 (segment (start 138.9617 88.575) (end 138.9617 89.4817) (width 0.2) (layer "B.Cu") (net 15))
 (segment (start 140.828 94.925) (end 138.8977 94.925) (width 0.2) (layer "B.Cu") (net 15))
 (segment (start 155 101.15) (end 153.9983 100.1483) (width 0.2) (layer "B.Cu") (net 15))
 (segment (start 138.8977 94.925) (end 138.0367 94.064) (width 0.2) (layer "B.Cu") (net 15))
 (segment (start 146.0513 100.1483) (end 140.828 94.925) (width 0.2) (layer "B.Cu") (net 15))
 (segment (start 138.0367 94.064) (end 138.0367 90.4067) (width 0.2) (layer "B.Cu") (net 15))
 (segment (start 156.0017 101.15) (end 155 101.15) (width 0.2) (layer "B.Cu") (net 15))
 (segment (start 138.9617 98.735) (end 145.5345 105.3078) (width 0.2) (layer "B.Cu") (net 2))
 (segment (start 145.5345 105.3078) (end 153.9922 105.3078) (width 0.2) (layer "B.Cu") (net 2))
 (segment (start 153.9922 105.3078) (end 155 104.3) (width 0.2) (layer "B.Cu") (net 2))
 (segment (start 156.0017 104.3) (end 155 104.3) (width 0.2) (layer "B.Cu") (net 2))
 (segment (start 150.2997 112.0121) (end 144.207 105.9194) (width 0.2) (layer "F.Cu") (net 3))
 (segment (start 156.0017 108.4517) (end 152.4413 112.0121) (width 0.2) (layer "F.Cu") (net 3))
 (segment (start 156.0017 107.45) (end 156.0017 108.4517) (width 0.2) (layer "F.Cu") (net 3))
 (segment (start 152.4413 112.0121) (end 150.2997 112.0121) (width 0.2) (layer "F.Cu") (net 3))
 (segment (start 144.207 105.9194) (end 144.207 96.3603) (width 0.2) (layer "F.Cu") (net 3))
 (segment (start 144.207 96.3603) (end 138.9617 91.115) (width 0.2) (layer "F.Cu") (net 3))
 (segment (start 138.9383 100.005) (end 138.0319 99.0986) (width 0.2) (layer "B.Cu") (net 5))
 (segment (start 153.1949 108.7949) (end 148.0221 108.7949) (width 0.2) (layer "B.Cu") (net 5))
 (segment (start 138.0319 97.1248) (end 138.9617 96.195) (width 0.2) (layer "B.Cu") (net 5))
 (segment (start 148.0221 108.7949) (end 139.2322 100.005) (width 0.2) (layer "B.Cu") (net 5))
 (segment (start 138.0319 99.0986) (end 138.0319 97.1248) (width 0.2) (layer "B.Cu") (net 5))
 (segment (start 156.0017 110.6) (end 155 110.6) (width 0.2) (layer "B.Cu") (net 5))
 (segment (start 155 110.6) (end 153.1949 108.7949) (width 0.2) (layer "B.Cu") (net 5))
 (segment (start 139.2322 100.005) (end 138.9383 100.005) (width 0.2) (layer "B.Cu") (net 5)))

